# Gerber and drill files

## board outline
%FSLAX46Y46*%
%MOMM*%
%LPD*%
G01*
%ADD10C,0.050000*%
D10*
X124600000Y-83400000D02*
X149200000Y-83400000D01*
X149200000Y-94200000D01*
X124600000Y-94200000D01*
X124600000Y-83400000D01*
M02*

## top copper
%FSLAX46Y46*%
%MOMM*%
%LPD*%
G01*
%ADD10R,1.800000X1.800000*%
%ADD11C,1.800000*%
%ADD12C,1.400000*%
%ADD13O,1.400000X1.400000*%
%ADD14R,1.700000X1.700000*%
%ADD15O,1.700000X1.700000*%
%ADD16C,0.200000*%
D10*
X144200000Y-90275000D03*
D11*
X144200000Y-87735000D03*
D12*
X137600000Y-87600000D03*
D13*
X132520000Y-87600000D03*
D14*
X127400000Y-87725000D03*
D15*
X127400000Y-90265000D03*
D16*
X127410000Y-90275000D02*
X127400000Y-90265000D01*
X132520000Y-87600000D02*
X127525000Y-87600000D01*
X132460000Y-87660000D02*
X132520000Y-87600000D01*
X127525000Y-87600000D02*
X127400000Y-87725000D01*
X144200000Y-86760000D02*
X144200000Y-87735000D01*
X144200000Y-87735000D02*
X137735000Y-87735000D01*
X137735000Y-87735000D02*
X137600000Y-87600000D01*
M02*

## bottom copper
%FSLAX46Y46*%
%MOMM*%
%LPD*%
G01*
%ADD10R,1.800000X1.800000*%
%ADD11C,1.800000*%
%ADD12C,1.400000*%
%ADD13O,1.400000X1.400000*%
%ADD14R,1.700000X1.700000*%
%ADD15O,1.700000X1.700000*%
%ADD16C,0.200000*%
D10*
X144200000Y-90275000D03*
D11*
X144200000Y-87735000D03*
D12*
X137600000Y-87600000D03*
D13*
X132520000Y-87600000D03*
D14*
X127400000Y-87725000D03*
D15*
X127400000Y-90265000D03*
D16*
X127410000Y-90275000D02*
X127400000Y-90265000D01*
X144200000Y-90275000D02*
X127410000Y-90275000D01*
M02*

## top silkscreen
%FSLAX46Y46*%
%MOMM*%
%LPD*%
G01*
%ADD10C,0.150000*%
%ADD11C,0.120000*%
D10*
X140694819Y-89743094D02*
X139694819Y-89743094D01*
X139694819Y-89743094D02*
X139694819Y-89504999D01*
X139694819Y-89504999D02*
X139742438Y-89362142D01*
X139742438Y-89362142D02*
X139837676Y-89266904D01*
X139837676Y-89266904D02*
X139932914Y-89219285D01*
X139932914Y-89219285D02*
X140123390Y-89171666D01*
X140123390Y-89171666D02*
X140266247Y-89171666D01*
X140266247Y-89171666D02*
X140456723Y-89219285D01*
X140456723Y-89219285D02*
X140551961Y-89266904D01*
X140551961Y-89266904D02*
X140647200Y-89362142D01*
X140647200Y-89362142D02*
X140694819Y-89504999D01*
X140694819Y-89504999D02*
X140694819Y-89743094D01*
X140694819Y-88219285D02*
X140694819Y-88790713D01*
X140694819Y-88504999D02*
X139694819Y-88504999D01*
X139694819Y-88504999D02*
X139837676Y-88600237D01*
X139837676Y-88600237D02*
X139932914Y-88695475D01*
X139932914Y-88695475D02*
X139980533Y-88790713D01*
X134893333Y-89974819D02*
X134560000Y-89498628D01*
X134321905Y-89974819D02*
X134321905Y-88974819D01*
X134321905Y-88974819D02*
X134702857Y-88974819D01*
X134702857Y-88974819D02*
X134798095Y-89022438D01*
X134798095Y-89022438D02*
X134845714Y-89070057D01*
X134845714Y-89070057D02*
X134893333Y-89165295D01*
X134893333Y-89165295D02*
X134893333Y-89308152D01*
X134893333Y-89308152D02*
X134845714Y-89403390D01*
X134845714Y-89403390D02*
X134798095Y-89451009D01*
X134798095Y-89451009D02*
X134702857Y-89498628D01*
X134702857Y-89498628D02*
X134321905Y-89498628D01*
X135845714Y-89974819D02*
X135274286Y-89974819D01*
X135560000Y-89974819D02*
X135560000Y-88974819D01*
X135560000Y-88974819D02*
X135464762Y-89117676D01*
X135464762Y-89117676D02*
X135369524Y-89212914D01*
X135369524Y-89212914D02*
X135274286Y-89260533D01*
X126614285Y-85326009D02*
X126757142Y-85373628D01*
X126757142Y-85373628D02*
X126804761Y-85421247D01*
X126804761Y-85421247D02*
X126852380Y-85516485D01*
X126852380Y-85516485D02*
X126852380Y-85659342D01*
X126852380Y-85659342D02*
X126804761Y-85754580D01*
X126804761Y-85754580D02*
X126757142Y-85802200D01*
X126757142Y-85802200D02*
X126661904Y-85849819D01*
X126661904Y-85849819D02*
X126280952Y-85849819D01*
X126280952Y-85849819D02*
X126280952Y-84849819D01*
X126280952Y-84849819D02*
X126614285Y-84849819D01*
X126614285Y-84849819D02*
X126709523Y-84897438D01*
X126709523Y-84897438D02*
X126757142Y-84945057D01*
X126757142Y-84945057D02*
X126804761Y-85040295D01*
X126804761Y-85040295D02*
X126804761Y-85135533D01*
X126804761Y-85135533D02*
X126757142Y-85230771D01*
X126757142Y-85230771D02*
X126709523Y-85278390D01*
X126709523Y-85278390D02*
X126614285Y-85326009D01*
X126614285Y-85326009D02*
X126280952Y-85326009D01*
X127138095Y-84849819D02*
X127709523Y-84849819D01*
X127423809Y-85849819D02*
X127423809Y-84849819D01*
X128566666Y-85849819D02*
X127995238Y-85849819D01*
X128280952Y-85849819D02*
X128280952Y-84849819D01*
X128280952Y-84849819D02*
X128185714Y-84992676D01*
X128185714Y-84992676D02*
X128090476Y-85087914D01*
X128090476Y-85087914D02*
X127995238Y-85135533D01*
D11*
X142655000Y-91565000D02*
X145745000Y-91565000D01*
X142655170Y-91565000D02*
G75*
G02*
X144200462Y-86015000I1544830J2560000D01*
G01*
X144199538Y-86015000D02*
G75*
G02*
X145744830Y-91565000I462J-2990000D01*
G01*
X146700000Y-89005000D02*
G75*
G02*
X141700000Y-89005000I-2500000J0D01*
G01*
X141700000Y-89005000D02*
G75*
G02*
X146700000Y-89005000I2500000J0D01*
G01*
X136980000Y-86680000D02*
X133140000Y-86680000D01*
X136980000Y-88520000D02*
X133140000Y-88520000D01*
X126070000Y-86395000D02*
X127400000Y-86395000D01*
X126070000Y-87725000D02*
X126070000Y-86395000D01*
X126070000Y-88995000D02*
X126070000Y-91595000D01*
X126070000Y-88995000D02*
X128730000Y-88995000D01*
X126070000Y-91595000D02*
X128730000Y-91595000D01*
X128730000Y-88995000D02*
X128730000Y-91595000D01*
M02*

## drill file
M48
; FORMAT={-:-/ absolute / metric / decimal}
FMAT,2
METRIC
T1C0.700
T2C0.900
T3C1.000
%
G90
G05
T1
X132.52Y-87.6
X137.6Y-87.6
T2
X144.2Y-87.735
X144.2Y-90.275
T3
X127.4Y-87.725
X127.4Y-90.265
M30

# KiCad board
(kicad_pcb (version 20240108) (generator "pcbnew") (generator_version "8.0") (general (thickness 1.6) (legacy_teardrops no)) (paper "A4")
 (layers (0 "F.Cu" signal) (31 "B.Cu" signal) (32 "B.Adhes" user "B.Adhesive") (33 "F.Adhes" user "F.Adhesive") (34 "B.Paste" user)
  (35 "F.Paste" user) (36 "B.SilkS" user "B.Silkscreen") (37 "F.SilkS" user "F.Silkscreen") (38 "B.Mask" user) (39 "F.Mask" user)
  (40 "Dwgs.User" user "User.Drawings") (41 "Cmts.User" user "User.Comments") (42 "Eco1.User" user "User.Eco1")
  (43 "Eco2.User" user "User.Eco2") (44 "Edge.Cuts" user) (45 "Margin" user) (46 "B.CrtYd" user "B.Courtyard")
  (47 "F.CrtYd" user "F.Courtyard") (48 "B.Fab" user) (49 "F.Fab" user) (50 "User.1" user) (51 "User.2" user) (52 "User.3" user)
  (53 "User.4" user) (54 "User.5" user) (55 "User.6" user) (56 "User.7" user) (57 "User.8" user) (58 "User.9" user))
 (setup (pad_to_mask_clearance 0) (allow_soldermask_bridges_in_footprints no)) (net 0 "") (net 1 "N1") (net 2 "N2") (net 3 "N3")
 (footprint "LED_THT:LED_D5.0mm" (layer "F.Cu") (at 144.2 90.275 90)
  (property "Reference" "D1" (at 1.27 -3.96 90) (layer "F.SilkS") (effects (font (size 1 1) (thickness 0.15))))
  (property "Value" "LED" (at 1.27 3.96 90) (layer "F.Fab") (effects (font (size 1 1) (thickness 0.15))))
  (fp_line (start -1.29 -1.545) (end -1.29 1.545) (stroke (width 0.12) (type solid)) (layer "F.SilkS"))
  (fp_arc (start -1.29 -1.54483) (mid 2.072002 -2.880433) (end 4.26 0.000462) (stroke (width 0.12) (type solid)) (layer "F.SilkS"))
  (fp_arc (start 4.26 -0.000462) (mid 2.072002 2.880433) (end -1.29 1.54483) (stroke (width 0.12) (type solid)) (layer "F.SilkS"))
  (fp_circle (center 1.27 0) (end 3.77 0) (stroke (width 0.12) (type solid)) (fill none) (layer "F.SilkS"))
  (pad "1" thru_hole rect (at 0 0 90) (size 1.8 1.8) (drill 0.9) (layers "*.Cu" "*.Mask") (remove_unused_layers no) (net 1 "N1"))
  (pad "2" thru_hole circle (at 2.54 0 90) (size 1.8 1.8) (drill 0.9) (layers "*.Cu" "*.Mask") (remove_unused_layers no) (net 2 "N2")))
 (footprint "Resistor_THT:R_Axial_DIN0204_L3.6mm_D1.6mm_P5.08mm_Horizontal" (layer "F.Cu") (at 137.6 87.6 180)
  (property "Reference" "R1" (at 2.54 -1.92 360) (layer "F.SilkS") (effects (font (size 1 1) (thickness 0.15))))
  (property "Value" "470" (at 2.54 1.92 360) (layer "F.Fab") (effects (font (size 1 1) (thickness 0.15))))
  (fp_line (start 0.62 0.92) (end 4.46 0.92) (stroke (width 0.12) (type solid)) (layer "F.SilkS"))
  (fp_line (start 0.62 -0.92) (end 4.46 -0.92) (stroke (width 0.12) (type solid)) (layer "F.SilkS"))
  (pad "1" thru_hole circle (at 0 0 180) (size 1.4 1.4) (drill 0.7) (layers "*.Cu" "*.Mask") (remove_unused_layers no) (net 2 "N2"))
  (pad "2" thru_hole oval (at 5.08 0 180) (size 1.4 1.4) (drill 0.7) (layers "*.Cu" "*.Mask") (remove_unused_layers no) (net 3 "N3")))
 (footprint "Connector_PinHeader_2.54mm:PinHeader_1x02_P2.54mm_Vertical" (layer "F.Cu") (at 127.4 87.725)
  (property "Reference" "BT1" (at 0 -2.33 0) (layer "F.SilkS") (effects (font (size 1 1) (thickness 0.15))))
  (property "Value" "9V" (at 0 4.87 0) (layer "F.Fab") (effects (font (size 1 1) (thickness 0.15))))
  (fp_line (start -1.33 -1.33) (end 0 -1.33) (stroke (width 0.12) (type solid)) (layer "F.SilkS"))
  (fp_line (start -1.33 0) (end -1.33 -1.33) (stroke (width 0.12) (type solid)) (layer "F.SilkS"))
  (fp_line (start -1.33 1.27) (end -1.33 3.87) (stroke (width 0.12) (type solid)) (layer "F.SilkS"))
  (fp_line (start -1.33 1.27) (end 1.33 1.27) (stroke (width 0.12) (type solid)) (layer "F.SilkS"))
  (fp_line (start -1.33 3.87) (end 1.33 3.87) (stroke (width 0.12) (type solid)) (layer "F.SilkS"))
  (fp_line (start 1.33 1.27) (end 1.33 3.87) (stroke (width 0.12) (type solid)) (layer "F.SilkS"))
  (pad "1" thru_hole rect (at 0 0) (size 1.7 1.7) (drill 1) (layers "*.Cu" "*.Mask") (remove_unused_layers no) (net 3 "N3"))
  (pad "2" thru_hole oval (at 0 2.54) (size 1.7 1.7) (drill 1) (layers "*.Cu" "*.Mask") (remove_unused_layers no) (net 1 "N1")))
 (gr_rect (start 124.6 83.4) (end 149.2 94.2) (stroke (width 0.05) (type default)) (fill none) (layer "Edge.Cuts"))
 (segment (start 127.41 90.275) (end 127.4 90.265) (width 0.2) (layer "F.Cu") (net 1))
 (segment (start 127.41 90.275) (end 127.4 90.265) (width 0.2) (layer "B.Cu") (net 1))
 (segment (start 144.2 90.275) (end 127.41 90.275) (width 0.2) (layer "B.Cu") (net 1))
 (segment (start 132.52 87.6) (end 127.525 87.6) (width 0.2) (layer "F.Cu") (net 3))
 (segment (start 132.46 87.66) (end 132.52 87.6) (width 0.2) (layer "F.Cu") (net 3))
 (segment (start 127.525 87.6) (end 127.4 87.725) (width 0.2) (layer "F.Cu") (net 3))
 (segment (start 144.2 86.76) (end 144.2 87.735) (width 0.2) (layer "F.Cu") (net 2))
 (segment (start 144.2 87.735) (end 137.735 87.735) (width 0.2) (layer "F.Cu") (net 2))
 (segment (start 137.735 87.735) (end 137.6 87.6) (width 0.2) (layer "F.Cu") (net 2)))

